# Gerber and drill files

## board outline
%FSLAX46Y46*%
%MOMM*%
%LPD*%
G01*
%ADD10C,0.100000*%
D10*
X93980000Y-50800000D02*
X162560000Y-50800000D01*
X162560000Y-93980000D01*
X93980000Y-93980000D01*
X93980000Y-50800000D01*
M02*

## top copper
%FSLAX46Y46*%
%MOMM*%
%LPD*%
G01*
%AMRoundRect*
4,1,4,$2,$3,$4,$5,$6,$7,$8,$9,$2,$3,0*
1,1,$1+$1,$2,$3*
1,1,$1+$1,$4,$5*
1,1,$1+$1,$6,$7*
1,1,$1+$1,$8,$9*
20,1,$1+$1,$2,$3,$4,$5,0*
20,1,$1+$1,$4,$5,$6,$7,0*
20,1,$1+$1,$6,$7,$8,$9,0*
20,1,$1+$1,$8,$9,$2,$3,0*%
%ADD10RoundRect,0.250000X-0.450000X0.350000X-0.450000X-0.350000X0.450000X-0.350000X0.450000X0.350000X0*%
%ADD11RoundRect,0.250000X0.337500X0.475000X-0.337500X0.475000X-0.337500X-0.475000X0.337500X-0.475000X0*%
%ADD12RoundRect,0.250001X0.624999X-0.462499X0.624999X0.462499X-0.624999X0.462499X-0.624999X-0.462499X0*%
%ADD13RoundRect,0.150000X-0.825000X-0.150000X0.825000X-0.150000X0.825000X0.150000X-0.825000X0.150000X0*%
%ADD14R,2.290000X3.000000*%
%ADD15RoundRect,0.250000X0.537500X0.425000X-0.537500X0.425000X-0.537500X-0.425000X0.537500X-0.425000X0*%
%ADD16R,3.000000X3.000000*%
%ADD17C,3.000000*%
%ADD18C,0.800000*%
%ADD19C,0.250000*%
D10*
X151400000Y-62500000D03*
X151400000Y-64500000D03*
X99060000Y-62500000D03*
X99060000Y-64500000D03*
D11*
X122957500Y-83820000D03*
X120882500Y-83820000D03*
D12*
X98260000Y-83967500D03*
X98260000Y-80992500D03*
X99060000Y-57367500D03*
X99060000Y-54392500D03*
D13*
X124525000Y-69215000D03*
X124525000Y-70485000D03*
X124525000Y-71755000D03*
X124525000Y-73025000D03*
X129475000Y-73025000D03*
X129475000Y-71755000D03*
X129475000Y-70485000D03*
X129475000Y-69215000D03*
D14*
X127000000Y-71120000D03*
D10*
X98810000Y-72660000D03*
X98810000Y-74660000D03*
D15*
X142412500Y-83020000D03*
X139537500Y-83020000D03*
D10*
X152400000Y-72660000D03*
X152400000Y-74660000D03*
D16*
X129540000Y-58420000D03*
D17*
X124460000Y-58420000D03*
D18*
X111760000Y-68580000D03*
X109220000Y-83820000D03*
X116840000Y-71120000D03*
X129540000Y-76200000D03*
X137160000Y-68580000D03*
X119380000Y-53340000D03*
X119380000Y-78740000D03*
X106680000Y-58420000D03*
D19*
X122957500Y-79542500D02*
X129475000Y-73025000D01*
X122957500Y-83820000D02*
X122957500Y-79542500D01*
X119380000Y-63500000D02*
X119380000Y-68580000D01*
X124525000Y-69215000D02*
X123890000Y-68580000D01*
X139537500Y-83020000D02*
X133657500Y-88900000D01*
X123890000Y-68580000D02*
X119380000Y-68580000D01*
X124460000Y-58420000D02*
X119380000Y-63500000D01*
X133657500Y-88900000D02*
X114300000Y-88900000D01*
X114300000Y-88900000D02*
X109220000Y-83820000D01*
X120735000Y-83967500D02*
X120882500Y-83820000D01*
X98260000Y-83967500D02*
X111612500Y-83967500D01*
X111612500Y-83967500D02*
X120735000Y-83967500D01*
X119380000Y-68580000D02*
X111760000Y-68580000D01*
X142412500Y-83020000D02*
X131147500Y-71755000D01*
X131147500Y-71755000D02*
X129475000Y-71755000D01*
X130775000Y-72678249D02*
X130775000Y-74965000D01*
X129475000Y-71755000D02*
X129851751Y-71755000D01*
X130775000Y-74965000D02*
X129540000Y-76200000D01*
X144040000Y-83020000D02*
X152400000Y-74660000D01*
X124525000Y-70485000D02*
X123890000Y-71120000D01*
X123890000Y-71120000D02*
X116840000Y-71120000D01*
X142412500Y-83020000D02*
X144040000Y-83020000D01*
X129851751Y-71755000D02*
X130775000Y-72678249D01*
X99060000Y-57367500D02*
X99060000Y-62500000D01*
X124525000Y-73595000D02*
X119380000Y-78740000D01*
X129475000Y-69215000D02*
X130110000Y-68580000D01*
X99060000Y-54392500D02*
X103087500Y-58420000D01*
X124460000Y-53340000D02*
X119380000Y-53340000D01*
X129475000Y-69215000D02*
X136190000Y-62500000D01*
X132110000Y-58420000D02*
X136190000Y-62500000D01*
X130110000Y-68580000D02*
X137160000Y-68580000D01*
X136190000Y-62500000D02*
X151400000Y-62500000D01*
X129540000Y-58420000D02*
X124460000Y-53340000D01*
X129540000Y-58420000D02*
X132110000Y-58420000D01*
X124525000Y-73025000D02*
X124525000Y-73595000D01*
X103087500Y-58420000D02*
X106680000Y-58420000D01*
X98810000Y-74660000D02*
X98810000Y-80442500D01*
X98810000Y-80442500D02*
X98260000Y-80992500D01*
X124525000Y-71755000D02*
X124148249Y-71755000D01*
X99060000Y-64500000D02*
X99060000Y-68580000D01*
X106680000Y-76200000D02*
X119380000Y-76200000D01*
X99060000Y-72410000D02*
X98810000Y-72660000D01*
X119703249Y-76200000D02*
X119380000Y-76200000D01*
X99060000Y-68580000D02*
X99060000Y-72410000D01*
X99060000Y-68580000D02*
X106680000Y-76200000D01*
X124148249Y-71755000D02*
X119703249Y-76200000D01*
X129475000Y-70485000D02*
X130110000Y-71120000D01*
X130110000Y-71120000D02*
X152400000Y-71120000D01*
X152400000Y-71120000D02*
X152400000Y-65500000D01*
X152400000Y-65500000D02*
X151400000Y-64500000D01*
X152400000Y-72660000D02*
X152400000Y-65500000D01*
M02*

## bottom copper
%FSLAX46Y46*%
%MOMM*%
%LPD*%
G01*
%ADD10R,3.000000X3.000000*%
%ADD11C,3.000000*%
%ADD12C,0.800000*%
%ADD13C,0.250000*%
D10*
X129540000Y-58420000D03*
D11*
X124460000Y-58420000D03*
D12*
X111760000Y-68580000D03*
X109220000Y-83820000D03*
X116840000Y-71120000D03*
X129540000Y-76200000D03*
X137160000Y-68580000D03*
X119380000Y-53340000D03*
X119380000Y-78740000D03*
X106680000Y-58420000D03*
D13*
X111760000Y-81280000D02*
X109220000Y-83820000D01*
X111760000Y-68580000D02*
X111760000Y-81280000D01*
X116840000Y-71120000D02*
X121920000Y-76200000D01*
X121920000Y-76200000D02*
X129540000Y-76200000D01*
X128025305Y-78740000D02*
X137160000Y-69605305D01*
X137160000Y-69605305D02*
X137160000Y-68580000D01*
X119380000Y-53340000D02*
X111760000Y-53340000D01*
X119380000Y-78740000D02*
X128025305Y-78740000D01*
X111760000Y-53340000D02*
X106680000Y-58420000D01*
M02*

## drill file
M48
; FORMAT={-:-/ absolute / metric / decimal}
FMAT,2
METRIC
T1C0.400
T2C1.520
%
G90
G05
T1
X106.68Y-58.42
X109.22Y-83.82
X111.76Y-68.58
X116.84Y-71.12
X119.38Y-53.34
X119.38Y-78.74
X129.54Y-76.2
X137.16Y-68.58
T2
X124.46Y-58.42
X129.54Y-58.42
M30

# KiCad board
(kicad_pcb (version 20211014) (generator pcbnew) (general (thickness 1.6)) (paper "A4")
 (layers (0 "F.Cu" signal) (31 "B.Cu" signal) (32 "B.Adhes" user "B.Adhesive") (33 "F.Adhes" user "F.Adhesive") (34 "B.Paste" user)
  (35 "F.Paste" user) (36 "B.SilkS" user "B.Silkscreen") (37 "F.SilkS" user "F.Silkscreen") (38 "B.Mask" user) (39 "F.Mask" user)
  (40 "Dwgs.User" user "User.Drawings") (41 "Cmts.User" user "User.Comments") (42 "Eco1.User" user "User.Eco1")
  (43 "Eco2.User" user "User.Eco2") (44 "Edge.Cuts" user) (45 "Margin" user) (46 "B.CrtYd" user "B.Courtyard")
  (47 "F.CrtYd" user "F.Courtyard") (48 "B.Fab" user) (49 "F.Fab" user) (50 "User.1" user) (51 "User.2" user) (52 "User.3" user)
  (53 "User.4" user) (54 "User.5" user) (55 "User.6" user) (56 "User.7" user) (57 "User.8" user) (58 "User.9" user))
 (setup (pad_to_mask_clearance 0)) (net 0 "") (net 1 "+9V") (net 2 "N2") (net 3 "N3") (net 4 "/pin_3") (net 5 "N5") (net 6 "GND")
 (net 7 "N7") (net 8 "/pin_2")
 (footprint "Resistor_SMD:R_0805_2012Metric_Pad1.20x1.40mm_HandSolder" (layer "F.Cu") (at 151.4 63.5 -90)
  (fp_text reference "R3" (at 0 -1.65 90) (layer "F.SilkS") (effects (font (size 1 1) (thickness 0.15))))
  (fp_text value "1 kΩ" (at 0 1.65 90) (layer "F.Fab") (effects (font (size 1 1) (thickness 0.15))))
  (pad "1" smd roundrect (at -1 0 270) (size 1.2 1.4) (layers "F.Cu" "F.Paste" "F.Mask") (roundrect_rratio 0.2083333333) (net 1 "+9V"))
  (pad "2" smd roundrect (at 1 0 270) (size 1.2 1.4) (layers "F.Cu" "F.Paste" "F.Mask") (roundrect_rratio 0.2083333333) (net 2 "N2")))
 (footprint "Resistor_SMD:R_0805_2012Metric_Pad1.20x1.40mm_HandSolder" (layer "F.Cu") (at 99.06 63.5 -90)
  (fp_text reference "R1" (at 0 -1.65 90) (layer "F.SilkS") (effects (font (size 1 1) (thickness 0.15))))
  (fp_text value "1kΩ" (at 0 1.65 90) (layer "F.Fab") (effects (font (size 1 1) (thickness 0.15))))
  (pad "1" smd roundrect (at -1 0 270) (size 1.2 1.4) (layers "F.Cu" "F.Paste" "F.Mask") (roundrect_rratio 0.2083333333) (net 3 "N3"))
  (pad "2" smd roundrect (at 1 0 270) (size 1.2 1.4) (layers "F.Cu" "F.Paste" "F.Mask") (roundrect_rratio 0.2083333333) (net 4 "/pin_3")))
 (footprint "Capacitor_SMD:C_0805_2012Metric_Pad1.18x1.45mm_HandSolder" (layer "F.Cu") (at 121.92 83.82 180)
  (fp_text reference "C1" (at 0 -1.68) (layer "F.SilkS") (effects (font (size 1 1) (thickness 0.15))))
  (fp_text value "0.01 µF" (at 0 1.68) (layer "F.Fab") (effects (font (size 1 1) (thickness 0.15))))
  (pad "1" smd roundrect (at -1.0375 0 180) (size 1.175 1.45) (layers "F.Cu" "F.Paste" "F.Mask") (roundrect_rratio 0.2127659574)
   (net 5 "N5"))
  (pad "2" smd roundrect (at 1.0375 0 180) (size 1.175 1.45) (layers "F.Cu" "F.Paste" "F.Mask") (roundrect_rratio 0.2127659574)
   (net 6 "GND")))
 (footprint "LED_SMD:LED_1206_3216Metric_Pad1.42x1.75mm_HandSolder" (layer "F.Cu") (at 98.26 82.48 90)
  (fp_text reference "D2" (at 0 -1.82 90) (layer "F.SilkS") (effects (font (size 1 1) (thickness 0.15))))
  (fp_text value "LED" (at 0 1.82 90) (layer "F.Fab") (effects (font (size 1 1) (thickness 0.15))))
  (pad "1" smd roundrect (at -1.4875 0 90) (size 1.425 1.75) (layers "F.Cu" "F.Paste" "F.Mask") (roundrect_rratio 0.1754392982)
   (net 6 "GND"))
  (pad "2" smd roundrect (at 1.4875 0 90) (size 1.425 1.75) (layers "F.Cu" "F.Paste" "F.Mask") (roundrect_rratio 0.1754392982) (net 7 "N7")))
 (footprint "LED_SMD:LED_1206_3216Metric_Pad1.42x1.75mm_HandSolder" (layer "F.Cu") (at 99.06 55.88 90)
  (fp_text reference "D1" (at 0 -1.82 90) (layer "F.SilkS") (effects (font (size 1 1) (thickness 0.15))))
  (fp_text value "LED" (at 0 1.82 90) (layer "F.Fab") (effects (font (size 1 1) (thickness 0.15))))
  (pad "1" smd roundrect (at -1.4875 0 90) (size 1.425 1.75) (layers "F.Cu" "F.Paste" "F.Mask") (roundrect_rratio 0.1754392982) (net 3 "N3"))
  (pad "2" smd roundrect (at 1.4875 0 90) (size 1.425 1.75) (layers "F.Cu" "F.Paste" "F.Mask") (roundrect_rratio 0.1754392982) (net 1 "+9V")))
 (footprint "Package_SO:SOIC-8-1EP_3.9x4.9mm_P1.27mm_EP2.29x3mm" (layer "F.Cu") (at 127 71.12)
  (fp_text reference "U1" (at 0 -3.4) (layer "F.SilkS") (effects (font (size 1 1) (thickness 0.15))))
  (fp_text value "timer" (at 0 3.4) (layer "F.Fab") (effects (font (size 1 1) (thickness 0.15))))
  (pad "" smd roundrect (at -0.57 0.75) (size 0.92 1.21) (layers "F.Paste") (roundrect_rratio 0.25))
  (pad "" smd roundrect (at 0.57 0.75) (size 0.92 1.21) (layers "F.Paste") (roundrect_rratio 0.25))
  (pad "" smd roundrect (at -0.57 -0.75) (size 0.92 1.21) (layers "F.Paste") (roundrect_rratio 0.25))
  (pad "" smd roundrect (at 0.57 -0.75) (size 0.92 1.21) (layers "F.Paste") (roundrect_rratio 0.25))
  (pad "1" smd roundrect (at -2.475 -1.905) (size 1.95 0.6) (layers "F.Cu" "F.Paste" "F.Mask") (roundrect_rratio 0.25) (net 6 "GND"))
  (pad "2" smd roundrect (at -2.475 -0.635) (size 1.95 0.6) (layers "F.Cu" "F.Paste" "F.Mask") (roundrect_rratio 0.25) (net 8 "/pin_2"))
  (pad "3" smd roundrect (at -2.475 0.635) (size 1.95 0.6) (layers "F.Cu" "F.Paste" "F.Mask") (roundrect_rratio 0.25) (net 4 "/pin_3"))
  (pad "4" smd roundrect (at -2.475 1.905) (size 1.95 0.6) (layers "F.Cu" "F.Paste" "F.Mask") (roundrect_rratio 0.25) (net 1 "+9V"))
  (pad "5" smd roundrect (at 2.475 1.905) (size 1.95 0.6) (layers "F.Cu" "F.Paste" "F.Mask") (roundrect_rratio 0.25) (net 5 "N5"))
  (pad "6" smd roundrect (at 2.475 0.635) (size 1.95 0.6) (layers "F.Cu" "F.Paste" "F.Mask") (roundrect_rratio 0.25) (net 8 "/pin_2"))
  (pad "7" smd roundrect (at 2.475 -0.635) (size 1.95 0.6) (layers "F.Cu" "F.Paste" "F.Mask") (roundrect_rratio 0.25) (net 2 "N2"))
  (pad "8" smd roundrect (at 2.475 -1.905) (size 1.95 0.6) (layers "F.Cu" "F.Paste" "F.Mask") (roundrect_rratio 0.25) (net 1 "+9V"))
  (pad "9" smd rect (at 0 0) (size 2.29 3) (layers "F.Cu" "F.Mask")))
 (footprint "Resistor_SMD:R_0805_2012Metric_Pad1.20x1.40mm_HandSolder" (layer "F.Cu") (at 98.81 73.66 -90)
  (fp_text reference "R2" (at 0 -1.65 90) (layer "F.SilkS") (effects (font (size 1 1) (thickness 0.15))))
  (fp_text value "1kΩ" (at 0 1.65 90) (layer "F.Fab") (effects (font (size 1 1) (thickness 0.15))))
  (pad "1" smd roundrect (at -1 0 270) (size 1.2 1.4) (layers "F.Cu" "F.Paste" "F.Mask") (roundrect_rratio 0.2083333333) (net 4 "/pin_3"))
  (pad "2" smd roundrect (at 1 0 270) (size 1.2 1.4) (layers "F.Cu" "F.Paste" "F.Mask") (roundrect_rratio 0.2083333333) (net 7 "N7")))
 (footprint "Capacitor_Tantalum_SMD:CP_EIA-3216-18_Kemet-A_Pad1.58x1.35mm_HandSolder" (layer "F.Cu") (at 140.975 83.02 180)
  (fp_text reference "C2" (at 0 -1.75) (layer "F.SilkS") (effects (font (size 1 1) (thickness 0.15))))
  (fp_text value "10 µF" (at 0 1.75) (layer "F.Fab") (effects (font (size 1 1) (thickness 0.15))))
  (pad "1" smd roundrect (at -1.4375 0 180) (size 1.575 1.35) (layers "F.Cu" "F.Paste" "F.Mask") (roundrect_rratio 0.1851851852)
   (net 8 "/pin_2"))
  (pad "2" smd roundrect (at 1.4375 0 180) (size 1.575 1.35) (layers "F.Cu" "F.Paste" "F.Mask") (roundrect_rratio 0.1851851852)
   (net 6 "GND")))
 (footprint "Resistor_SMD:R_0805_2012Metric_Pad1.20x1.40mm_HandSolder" (layer "F.Cu") (at 152.4 73.66 -90)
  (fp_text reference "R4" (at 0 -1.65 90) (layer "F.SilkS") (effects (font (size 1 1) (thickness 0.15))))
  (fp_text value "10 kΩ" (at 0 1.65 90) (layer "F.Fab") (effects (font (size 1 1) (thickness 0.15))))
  (pad "1" smd roundrect (at -1 0 270) (size 1.2 1.4) (layers "F.Cu" "F.Paste" "F.Mask") (roundrect_rratio 0.2083333333) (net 2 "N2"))
  (pad "2" smd roundrect (at 1 0 270) (size 1.2 1.4) (layers "F.Cu" "F.Paste" "F.Mask") (roundrect_rratio 0.2083333333) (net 8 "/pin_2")))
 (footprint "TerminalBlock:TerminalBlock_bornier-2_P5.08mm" (layer "F.Cu") (at 129.54 58.42 180)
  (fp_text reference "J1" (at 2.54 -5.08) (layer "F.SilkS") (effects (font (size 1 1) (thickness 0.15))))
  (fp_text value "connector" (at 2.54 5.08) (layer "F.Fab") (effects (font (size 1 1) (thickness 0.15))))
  (pad "1" thru_hole rect (at 0 0 180) (size 3 3) (drill 1.52) (layers *.Cu *.Mask) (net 1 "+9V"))
  (pad "2" thru_hole circle (at 5.08 0 180) (size 3 3) (drill 1.52) (layers *.Cu *.Mask) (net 6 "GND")))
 (gr_rect (start 93.98 50.8) (end 162.56 93.98) (layer "Edge.Cuts") (width 0.1) (fill none))
 (segment (start 122.9575 79.5425) (end 129.475 73.025) (width 0.25) (layer "F.Cu") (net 5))
 (segment (start 122.9575 83.82) (end 122.9575 79.5425) (width 0.25) (layer "F.Cu") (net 5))
 (segment (start 119.38 63.5) (end 119.38 68.58) (width 0.25) (layer "F.Cu") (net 6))
 (segment (start 124.525 69.215) (end 123.89 68.58) (width 0.25) (layer "F.Cu") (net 6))
 (segment (start 139.5375 83.02) (end 133.6575 88.9) (width 0.25) (layer "F.Cu") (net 6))
 (segment (start 123.89 68.58) (end 119.38 68.58) (width 0.25) (layer "F.Cu") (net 6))
 (segment (start 124.46 58.42) (end 119.38 63.5) (width 0.25) (layer "F.Cu") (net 6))
 (segment (start 133.6575 88.9) (end 114.3 88.9) (width 0.25) (layer "F.Cu") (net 6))
 (segment (start 114.3 88.9) (end 109.22 83.82) (width 0.25) (layer "F.Cu") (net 6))
 (segment (start 120.735 83.9675) (end 120.8825 83.82) (width 0.25) (layer "F.Cu") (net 6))
 (segment (start 98.26 83.9675) (end 111.6125 83.9675) (width 0.25) (layer "F.Cu") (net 6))
 (segment (start 111.6125 83.9675) (end 120.735 83.9675) (width 0.25) (layer "F.Cu") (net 6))
 (segment (start 119.38 68.58) (end 111.76 68.58) (width 0.25) (layer "F.Cu") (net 6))
 (via (at 111.76 68.58) (size 0.8) (drill 0.4) (layers "F.Cu" "B.Cu") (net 6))
 (via (at 109.22 83.82) (size 0.8) (drill 0.4) (layers "F.Cu" "B.Cu") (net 6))
 (segment (start 111.76 81.28) (end 109.22 83.82) (width 0.25) (layer "B.Cu") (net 6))
 (segment (start 111.76 68.58) (end 111.76 81.28) (width 0.25) (layer "B.Cu") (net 6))
 (segment (start 142.4125 83.02) (end 131.1475 71.755) (width 0.25) (layer "F.Cu") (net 8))
 (segment (start 131.1475 71.755) (end 129.475 71.755) (width 0.25) (layer "F.Cu") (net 8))
 (segment (start 130.775 72.678249) (end 130.775 74.965) (width 0.25) (layer "F.Cu") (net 8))
 (segment (start 129.475 71.755) (end 129.851751 71.755) (width 0.25) (layer "F.Cu") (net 8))
 (segment (start 130.775 74.965) (end 129.54 76.2) (width 0.25) (layer "F.Cu") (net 8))
 (segment (start 144.04 83.02) (end 152.4 74.66) (width 0.25) (layer "F.Cu") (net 8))
 (segment (start 124.525 70.485) (end 123.89 71.12) (width 0.25) (layer "F.Cu") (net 8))
 (segment (start 123.89 71.12) (end 116.84 71.12) (width 0.25) (layer "F.Cu") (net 8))
 (segment (start 142.4125 83.02) (end 144.04 83.02) (width 0.25) (layer "F.Cu") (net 8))
 (segment (start 129.851751 71.755) (end 130.775 72.678249) (width 0.25) (layer "F.Cu") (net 8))
 (via (at 116.84 71.12) (size 0.8) (drill 0.4) (layers "F.Cu" "B.Cu") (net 8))
 (via (at 129.54 76.2) (size 0.8) (drill 0.4) (layers "F.Cu" "B.Cu") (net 8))
 (segment (start 116.84 71.12) (end 121.92 76.2) (width 0.25) (layer "B.Cu") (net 8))
 (segment (start 121.92 76.2) (end 129.54 76.2) (width 0.25) (layer "B.Cu") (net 8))
 (segment (start 99.06 57.3675) (end 99.06 62.5) (width 0.25) (layer "F.Cu") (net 3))
 (segment (start 124.525 73.595) (end 119.38 78.74) (width 0.25) (layer "F.Cu") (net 1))
 (segment (start 129.475 69.215) (end 130.11 68.58) (width 0.25) (layer "F.Cu") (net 1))
 (segment (start 99.06 54.3925) (end 103.0875 58.42) (width 0.25) (layer "F.Cu") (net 1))
 (segment (start 124.46 53.34) (end 119.38 53.34) (width 0.25) (layer "F.Cu") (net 1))
 (segment (start 129.475 69.215) (end 136.19 62.5) (width 0.25) (layer "F.Cu") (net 1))
 (segment (start 132.11 58.42) (end 136.19 62.5) (width 0.25) (layer "F.Cu") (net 1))
 (segment (start 130.11 68.58) (end 137.16 68.58) (width 0.25) (layer "F.Cu") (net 1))
 (segment (start 136.19 62.5) (end 151.4 62.5) (width 0.25) (layer "F.Cu") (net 1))
 (segment (start 129.54 58.42) (end 124.46 53.34) (width 0.25) (layer "F.Cu") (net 1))
 (segment (start 129.54 58.42) (end 132.11 58.42) (width 0.25) (layer "F.Cu") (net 1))
 (segment (start 124.525 73.025) (end 124.525 73.595) (width 0.25) (layer "F.Cu") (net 1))
 (segment (start 103.0875 58.42) (end 106.68 58.42) (width 0.25) (layer "F.Cu") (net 1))
 (via (at 137.16 68.58) (size 0.8) (drill 0.4) (layers "F.Cu" "B.Cu") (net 1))
 (via (at 119.38 53.34) (size 0.8) (drill 0.4) (layers "F.Cu" "B.Cu") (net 1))
 (via (at 119.38 78.74) (size 0.8) (drill 0.4) (layers "F.Cu" "B.Cu") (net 1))
 (via (at 106.68 58.42) (size 0.8) (drill 0.4) (layers "F.Cu" "B.Cu") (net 1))
 (segment (start 128.025305 78.74) (end 137.16 69.605305) (width 0.25) (layer "B.Cu") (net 1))
 (segment (start 137.16 69.605305) (end 137.16 68.58) (width 0.25) (layer "B.Cu") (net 1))
 (segment (start 119.38 53.34) (end 111.76 53.34) (width 0.25) (layer "B.Cu") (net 1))
 (segment (start 119.38 78.74) (end 128.025305 78.74) (width 0.25) (layer "B.Cu") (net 1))
 (segment (start 111.76 53.34) (end 106.68 58.42) (width 0.25) (layer "B.Cu") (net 1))
 (segment (start 98.81 74.66) (end 98.81 80.4425) (width 0.25) (layer "F.Cu") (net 7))
 (segment (start 98.81 80.4425) (end 98.26 80.9925) (width 0.25) (layer "F.Cu") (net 7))
 (segment (start 124.525 71.755) (end 124.148249 71.755) (width 0.25) (layer "F.Cu") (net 4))
 (segment (start 99.06 64.5) (end 99.06 68.58) (width 0.25) (layer "F.Cu") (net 4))
 (segment (start 106.68 76.2) (end 119.38 76.2) (width 0.25) (layer "F.Cu") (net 4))
 (segment (start 99.06 72.41) (end 98.81 72.66) (width 0.25) (layer "F.Cu") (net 4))
 (segment (start 119.703249 76.2) (end 119.38 76.2) (width 0.25) (layer "F.Cu") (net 4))
 (segment (start 99.06 68.58) (end 99.06 72.41) (width 0.25) (layer "F.Cu") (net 4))
 (segment (start 99.06 68.58) (end 106.68 76.2) (width 0.25) (layer "F.Cu") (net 4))
 (segment (start 124.148249 71.755) (end 119.703249 76.2) (width 0.25) (layer "F.Cu") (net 4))
 (segment (start 129.475 70.485) (end 130.11 71.12) (width 0.25) (layer "F.Cu") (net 2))
 (segment (start 130.11 71.12) (end 152.4 71.12) (width 0.25) (layer "F.Cu") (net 2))
 (segment (start 152.4 71.12) (end 152.4 65.5) (width 0.25) (layer "F.Cu") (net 2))
 (segment (start 152.4 65.5) (end 151.4 64.5) (width 0.25) (layer "F.Cu") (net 2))
 (segment (start 152.4 72.66) (end 152.4 65.5) (width 0.25) (layer "F.Cu") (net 2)))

